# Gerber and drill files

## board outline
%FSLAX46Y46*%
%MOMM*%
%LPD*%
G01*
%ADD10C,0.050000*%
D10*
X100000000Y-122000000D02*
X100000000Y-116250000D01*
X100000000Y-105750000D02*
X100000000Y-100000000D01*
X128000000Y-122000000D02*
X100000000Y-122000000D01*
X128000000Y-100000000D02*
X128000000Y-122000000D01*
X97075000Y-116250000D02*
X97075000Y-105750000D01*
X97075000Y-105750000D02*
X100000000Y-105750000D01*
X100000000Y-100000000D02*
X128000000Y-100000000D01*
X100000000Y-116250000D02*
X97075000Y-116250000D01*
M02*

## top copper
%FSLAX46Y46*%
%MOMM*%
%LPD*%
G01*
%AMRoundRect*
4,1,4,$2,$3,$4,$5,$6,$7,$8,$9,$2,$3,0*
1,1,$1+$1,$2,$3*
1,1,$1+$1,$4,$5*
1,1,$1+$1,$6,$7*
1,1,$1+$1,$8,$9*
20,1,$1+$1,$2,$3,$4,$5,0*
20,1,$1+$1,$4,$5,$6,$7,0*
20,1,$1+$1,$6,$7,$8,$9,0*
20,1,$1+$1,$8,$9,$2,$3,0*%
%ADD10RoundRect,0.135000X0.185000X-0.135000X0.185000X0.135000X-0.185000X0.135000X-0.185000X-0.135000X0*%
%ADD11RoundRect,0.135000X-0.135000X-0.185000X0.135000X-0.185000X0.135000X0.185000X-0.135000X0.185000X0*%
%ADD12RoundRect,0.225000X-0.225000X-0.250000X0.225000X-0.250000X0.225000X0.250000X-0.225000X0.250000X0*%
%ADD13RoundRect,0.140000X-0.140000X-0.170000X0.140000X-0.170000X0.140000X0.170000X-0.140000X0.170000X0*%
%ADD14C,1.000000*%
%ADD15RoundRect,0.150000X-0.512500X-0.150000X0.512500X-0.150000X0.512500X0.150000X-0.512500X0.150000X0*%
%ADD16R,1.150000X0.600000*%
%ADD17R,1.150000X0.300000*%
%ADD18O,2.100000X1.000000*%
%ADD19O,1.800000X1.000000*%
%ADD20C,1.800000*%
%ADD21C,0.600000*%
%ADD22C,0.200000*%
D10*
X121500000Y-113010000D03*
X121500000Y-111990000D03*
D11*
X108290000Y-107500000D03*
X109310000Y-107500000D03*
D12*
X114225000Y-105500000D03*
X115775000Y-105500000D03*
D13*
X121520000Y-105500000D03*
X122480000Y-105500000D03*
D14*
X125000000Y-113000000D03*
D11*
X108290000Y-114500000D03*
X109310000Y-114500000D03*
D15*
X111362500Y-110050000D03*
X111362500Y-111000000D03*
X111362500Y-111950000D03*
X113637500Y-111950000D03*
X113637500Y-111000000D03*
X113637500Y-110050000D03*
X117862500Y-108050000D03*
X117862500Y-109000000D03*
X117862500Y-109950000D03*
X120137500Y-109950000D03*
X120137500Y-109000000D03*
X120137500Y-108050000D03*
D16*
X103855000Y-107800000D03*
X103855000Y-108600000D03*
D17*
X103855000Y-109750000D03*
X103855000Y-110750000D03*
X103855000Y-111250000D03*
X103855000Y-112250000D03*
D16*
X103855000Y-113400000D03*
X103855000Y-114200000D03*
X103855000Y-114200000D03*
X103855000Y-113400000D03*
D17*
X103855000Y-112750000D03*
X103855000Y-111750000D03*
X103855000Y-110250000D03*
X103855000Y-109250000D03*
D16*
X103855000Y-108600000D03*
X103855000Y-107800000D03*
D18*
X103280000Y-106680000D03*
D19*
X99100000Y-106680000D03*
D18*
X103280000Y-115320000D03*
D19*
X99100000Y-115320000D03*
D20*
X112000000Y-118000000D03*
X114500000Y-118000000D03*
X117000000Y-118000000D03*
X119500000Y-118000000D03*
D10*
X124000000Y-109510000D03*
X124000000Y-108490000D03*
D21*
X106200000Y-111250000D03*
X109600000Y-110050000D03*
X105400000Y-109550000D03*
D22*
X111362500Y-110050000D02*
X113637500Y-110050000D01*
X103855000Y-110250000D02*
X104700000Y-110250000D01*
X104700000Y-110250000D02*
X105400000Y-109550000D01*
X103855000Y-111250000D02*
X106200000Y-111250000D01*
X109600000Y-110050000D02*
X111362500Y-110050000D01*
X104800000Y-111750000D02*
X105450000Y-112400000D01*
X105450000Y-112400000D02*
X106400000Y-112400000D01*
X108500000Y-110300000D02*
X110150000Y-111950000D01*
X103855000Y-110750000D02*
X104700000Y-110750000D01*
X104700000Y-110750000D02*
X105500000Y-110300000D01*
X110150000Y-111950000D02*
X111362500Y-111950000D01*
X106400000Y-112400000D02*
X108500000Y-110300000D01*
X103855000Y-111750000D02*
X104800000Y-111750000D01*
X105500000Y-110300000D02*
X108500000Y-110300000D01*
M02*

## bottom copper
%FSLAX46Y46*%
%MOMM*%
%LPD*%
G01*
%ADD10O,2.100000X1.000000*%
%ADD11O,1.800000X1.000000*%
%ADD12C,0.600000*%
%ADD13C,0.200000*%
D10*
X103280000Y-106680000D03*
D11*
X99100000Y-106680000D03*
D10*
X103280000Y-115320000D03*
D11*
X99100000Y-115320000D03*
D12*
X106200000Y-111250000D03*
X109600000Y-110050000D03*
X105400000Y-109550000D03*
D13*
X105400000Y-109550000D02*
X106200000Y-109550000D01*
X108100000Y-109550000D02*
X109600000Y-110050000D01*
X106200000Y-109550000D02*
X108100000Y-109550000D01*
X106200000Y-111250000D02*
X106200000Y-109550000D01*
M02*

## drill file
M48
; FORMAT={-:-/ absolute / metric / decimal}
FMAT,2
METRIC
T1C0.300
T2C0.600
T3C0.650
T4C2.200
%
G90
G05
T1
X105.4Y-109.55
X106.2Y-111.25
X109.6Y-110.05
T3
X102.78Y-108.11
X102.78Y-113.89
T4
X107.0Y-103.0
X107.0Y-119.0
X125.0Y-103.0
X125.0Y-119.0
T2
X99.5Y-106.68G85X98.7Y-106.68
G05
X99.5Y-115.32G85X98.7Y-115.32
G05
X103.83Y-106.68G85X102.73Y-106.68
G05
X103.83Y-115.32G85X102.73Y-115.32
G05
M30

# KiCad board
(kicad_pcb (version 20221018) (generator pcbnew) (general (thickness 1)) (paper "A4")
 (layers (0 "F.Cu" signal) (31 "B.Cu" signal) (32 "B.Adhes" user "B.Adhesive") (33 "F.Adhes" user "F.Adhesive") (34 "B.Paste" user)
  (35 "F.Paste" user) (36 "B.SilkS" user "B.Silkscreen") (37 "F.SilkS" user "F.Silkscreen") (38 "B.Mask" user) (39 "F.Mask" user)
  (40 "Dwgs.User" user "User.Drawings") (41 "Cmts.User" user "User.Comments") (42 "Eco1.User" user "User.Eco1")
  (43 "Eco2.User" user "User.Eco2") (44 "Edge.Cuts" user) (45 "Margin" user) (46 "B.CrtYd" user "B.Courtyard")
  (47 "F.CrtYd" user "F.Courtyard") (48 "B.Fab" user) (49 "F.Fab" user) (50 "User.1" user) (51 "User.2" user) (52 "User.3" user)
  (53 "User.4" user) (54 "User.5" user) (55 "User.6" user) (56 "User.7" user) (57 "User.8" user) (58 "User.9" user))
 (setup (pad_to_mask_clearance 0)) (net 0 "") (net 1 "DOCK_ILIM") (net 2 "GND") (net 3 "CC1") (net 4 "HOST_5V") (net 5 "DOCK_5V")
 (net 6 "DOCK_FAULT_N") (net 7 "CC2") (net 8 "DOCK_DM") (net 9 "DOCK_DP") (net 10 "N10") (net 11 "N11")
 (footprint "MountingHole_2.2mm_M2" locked (layer "F.Cu") (at 107 119)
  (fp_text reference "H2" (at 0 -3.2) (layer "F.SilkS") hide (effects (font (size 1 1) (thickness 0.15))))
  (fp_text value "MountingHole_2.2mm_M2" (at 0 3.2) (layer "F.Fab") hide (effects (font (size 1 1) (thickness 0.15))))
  (pad "" np_thru_hole circle locked (at 0 0) (size 2.2 2.2) (drill 2.2) (layers "*.Cu" "*.Mask")))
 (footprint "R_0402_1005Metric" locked (layer "F.Cu") (at 121.5 112.5 90)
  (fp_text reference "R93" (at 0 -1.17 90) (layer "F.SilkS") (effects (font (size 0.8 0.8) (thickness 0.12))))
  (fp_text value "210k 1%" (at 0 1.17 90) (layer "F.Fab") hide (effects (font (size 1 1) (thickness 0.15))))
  (pad "1" smd roundrect locked (at -0.51 0 90) (size 0.54 0.64) (layers "F.Cu" "F.Paste" "F.Mask") (roundrect_rratio 0.25)
   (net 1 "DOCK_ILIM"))
  (pad "2" smd roundrect locked (at 0.51 0 90) (size 0.54 0.64) (layers "F.Cu" "F.Paste" "F.Mask") (roundrect_rratio 0.25) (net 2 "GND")))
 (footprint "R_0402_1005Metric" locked (layer "F.Cu") (at 108.8 107.5)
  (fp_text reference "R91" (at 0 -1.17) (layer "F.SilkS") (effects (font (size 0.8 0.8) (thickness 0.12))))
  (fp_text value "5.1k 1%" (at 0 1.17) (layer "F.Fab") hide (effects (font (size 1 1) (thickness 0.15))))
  (pad "1" smd roundrect locked (at -0.51 0) (size 0.54 0.64) (layers "F.Cu" "F.Paste" "F.Mask") (roundrect_rratio 0.25) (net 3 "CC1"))
  (pad "2" smd roundrect locked (at 0.51 0) (size 0.54 0.64) (layers "F.Cu" "F.Paste" "F.Mask") (roundrect_rratio 0.25) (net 2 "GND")))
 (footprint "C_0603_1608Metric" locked (layer "F.Cu") (at 115 105.5)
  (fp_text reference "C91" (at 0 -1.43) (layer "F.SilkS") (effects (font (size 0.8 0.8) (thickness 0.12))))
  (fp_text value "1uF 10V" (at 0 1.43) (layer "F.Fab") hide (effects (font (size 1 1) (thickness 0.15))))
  (pad "1" smd roundrect locked (at -0.775 0) (size 0.9 0.95) (layers "F.Cu" "F.Paste" "F.Mask") (roundrect_rratio 0.25) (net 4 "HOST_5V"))
  (pad "2" smd roundrect locked (at 0.775 0) (size 0.9 0.95) (layers "F.Cu" "F.Paste" "F.Mask") (roundrect_rratio 0.25) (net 2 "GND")))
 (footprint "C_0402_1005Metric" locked (layer "F.Cu") (at 122 105.5)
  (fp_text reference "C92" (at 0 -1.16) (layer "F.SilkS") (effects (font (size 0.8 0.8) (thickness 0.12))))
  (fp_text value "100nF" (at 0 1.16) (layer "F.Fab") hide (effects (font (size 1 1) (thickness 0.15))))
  (pad "1" smd roundrect locked (at -0.48 0) (size 0.56 0.62) (layers "F.Cu" "F.Paste" "F.Mask") (roundrect_rratio 0.25) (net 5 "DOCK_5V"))
  (pad "2" smd roundrect locked (at 0.48 0) (size 0.56 0.62) (layers "F.Cu" "F.Paste" "F.Mask") (roundrect_rratio 0.25) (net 2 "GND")))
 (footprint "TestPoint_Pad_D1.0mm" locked (layer "F.Cu") (at 125 113)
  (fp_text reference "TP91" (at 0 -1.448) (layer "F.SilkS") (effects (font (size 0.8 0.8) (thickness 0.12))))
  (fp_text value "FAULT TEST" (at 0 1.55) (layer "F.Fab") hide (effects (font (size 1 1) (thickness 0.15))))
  (pad "1" smd circle locked (at 0 0) (size 1 1) (layers "F.Cu" "F.Mask") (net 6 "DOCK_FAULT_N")))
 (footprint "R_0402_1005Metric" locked (layer "F.Cu") (at 108.8 114.5)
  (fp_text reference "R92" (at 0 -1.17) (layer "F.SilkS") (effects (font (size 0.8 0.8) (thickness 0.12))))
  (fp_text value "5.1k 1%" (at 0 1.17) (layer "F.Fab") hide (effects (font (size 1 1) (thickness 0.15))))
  (pad "1" smd roundrect locked (at -0.51 0) (size 0.54 0.64) (layers "F.Cu" "F.Paste" "F.Mask") (roundrect_rratio 0.25) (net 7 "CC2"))
  (pad "2" smd roundrect locked (at 0.51 0) (size 0.54 0.64) (layers "F.Cu" "F.Paste" "F.Mask") (roundrect_rratio 0.25) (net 2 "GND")))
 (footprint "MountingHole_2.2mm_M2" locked (layer "F.Cu") (at 107 103)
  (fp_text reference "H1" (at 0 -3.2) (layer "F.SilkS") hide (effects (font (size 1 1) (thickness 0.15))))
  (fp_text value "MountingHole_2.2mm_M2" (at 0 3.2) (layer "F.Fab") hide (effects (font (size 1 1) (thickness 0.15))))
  (pad "" np_thru_hole circle locked (at 0 0) (size 2.2 2.2) (drill 2.2) (layers "*.Cu" "*.Mask")))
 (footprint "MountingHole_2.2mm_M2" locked (layer "F.Cu") (at 125 119)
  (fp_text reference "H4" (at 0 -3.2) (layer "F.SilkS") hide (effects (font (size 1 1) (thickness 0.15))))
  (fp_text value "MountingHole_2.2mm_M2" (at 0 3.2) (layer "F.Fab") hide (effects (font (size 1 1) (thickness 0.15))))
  (pad "" np_thru_hole circle locked (at 0 0) (size 2.2 2.2) (drill 2.2) (layers "*.Cu" "*.Mask")))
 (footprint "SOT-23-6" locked (layer "F.Cu") (at 112.5 111)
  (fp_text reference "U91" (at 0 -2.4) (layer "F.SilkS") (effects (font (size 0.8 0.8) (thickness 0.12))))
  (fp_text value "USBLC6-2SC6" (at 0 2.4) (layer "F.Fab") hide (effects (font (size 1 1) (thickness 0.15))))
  (pad "1" smd roundrect locked (at -1.1375 -0.95) (size 1.325 0.6) (layers "F.Cu" "F.Paste" "F.Mask") (roundrect_rratio 0.25)
   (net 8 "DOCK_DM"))
  (pad "2" smd roundrect locked (at -1.1375 0) (size 1.325 0.6) (layers "F.Cu" "F.Paste" "F.Mask") (roundrect_rratio 0.25) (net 2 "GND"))
  (pad "3" smd roundrect locked (at -1.1375 0.95) (size 1.325 0.6) (layers "F.Cu" "F.Paste" "F.Mask") (roundrect_rratio 0.25)
   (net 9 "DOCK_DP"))
  (pad "4" smd roundrect locked (at 1.1375 0.95) (size 1.325 0.6) (layers "F.Cu" "F.Paste" "F.Mask") (roundrect_rratio 0.25)
   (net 9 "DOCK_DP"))
  (pad "5" smd roundrect locked (at 1.1375 0) (size 1.325 0.6) (layers "F.Cu" "F.Paste" "F.Mask") (roundrect_rratio 0.25) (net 4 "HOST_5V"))
  (pad "6" smd roundrect locked (at 1.1375 -0.95) (size 1.325 0.6) (layers "F.Cu" "F.Paste" "F.Mask") (roundrect_rratio 0.25)
   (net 8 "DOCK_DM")))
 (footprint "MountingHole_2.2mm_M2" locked (layer "F.Cu") (at 125 103)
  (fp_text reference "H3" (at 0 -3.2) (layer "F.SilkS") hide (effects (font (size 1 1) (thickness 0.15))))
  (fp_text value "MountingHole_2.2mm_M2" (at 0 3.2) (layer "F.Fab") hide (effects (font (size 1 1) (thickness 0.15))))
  (pad "" np_thru_hole circle locked (at 0 0) (size 2.2 2.2) (drill 2.2) (layers "*.Cu" "*.Mask")))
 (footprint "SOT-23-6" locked (layer "F.Cu") (at 119 109)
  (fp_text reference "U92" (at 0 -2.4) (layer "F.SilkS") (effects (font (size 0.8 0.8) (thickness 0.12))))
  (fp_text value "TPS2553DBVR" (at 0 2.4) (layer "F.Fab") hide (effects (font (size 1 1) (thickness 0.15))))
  (pad "1" smd roundrect locked (at -1.1375 -0.95) (size 1.325 0.6) (layers "F.Cu" "F.Paste" "F.Mask") (roundrect_rratio 0.25)
   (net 4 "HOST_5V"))
  (pad "2" smd roundrect locked (at -1.1375 0) (size 1.325 0.6) (layers "F.Cu" "F.Paste" "F.Mask") (roundrect_rratio 0.25) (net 2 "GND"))
  (pad "3" smd roundrect locked (at -1.1375 0.95) (size 1.325 0.6) (layers "F.Cu" "F.Paste" "F.Mask") (roundrect_rratio 0.25)
   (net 4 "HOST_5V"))
  (pad "4" smd roundrect locked (at 1.1375 0.95) (size 1.325 0.6) (layers "F.Cu" "F.Paste" "F.Mask") (roundrect_rratio 0.25)
   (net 6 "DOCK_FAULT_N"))
  (pad "5" smd roundrect locked (at 1.1375 0) (size 1.325 0.6) (layers "F.Cu" "F.Paste" "F.Mask") (roundrect_rratio 0.25)
   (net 1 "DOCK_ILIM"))
  (pad "6" smd roundrect locked (at 1.1375 -0.95) (size 1.325 0.6) (layers "F.Cu" "F.Paste" "F.Mask") (roundrect_rratio 0.25)
   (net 5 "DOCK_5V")))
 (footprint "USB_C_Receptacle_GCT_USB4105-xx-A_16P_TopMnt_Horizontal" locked (layer "F.Cu") (at 100.175 111 -90)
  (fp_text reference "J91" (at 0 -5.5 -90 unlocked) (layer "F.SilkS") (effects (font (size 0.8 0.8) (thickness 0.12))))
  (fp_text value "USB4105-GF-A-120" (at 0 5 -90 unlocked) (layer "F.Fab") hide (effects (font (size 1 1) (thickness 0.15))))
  (pad "" np_thru_hole circle locked (at -2.89 -2.605 270) (size 0.65 0.65) (drill 0.65) (layers "F&B.Cu" "*.Mask"))
  (pad "" np_thru_hole circle locked (at 2.89 -2.605 270) (size 0.65 0.65) (drill 0.65) (layers "F&B.Cu" "*.Mask"))
  (pad "A1" smd rect locked (at -3.2 -3.68 270) (size 0.6 1.15) (layers "F.Cu" "F.Paste" "F.Mask") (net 2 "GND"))
  (pad "A4" smd rect locked (at -2.4 -3.68 270) (size 0.6 1.15) (layers "F.Cu" "F.Paste" "F.Mask") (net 4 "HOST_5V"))
  (pad "A5" smd rect locked (at -1.25 -3.68 270) (size 0.3 1.15) (layers "F.Cu" "F.Paste" "F.Mask") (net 3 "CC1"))
  (pad "A6" smd rect locked (at -0.25 -3.68 270) (size 0.3 1.15) (layers "F.Cu" "F.Paste" "F.Mask") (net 9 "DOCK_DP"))
  (pad "A7" smd rect locked (at 0.25 -3.68 270) (size 0.3 1.15) (layers "F.Cu" "F.Paste" "F.Mask") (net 8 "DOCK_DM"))
  (pad "A8" smd rect locked (at 1.25 -3.68 270) (size 0.3 1.15) (layers "F.Cu" "F.Paste" "F.Mask") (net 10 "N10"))
  (pad "A9" smd rect locked (at 2.4 -3.68 270) (size 0.6 1.15) (layers "F.Cu" "F.Paste" "F.Mask") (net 4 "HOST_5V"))
  (pad "A12" smd rect locked (at 3.2 -3.68 270) (size 0.6 1.15) (layers "F.Cu" "F.Paste" "F.Mask") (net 2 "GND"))
  (pad "B1" smd rect locked (at 3.2 -3.68 270) (size 0.6 1.15) (layers "F.Cu" "F.Paste" "F.Mask") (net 2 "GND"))
  (pad "B4" smd rect locked (at 2.4 -3.68 270) (size 0.6 1.15) (layers "F.Cu" "F.Paste" "F.Mask") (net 4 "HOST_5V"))
  (pad "B5" smd rect locked (at 1.75 -3.68 270) (size 0.3 1.15) (layers "F.Cu" "F.Paste" "F.Mask") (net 7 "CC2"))
  (pad "B6" smd rect locked (at 0.75 -3.68 270) (size 0.3 1.15) (layers "F.Cu" "F.Paste" "F.Mask") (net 9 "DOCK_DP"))
  (pad "B7" smd rect locked (at -0.75 -3.68 270) (size 0.3 1.15) (layers "F.Cu" "F.Paste" "F.Mask") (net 8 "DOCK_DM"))
  (pad "B8" smd rect locked (at -1.75 -3.68 270) (size 0.3 1.15) (layers "F.Cu" "F.Paste" "F.Mask") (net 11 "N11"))
  (pad "B9" smd rect locked (at -2.4 -3.68 270) (size 0.6 1.15) (layers "F.Cu" "F.Paste" "F.Mask") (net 4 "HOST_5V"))
  (pad "B12" smd rect locked (at -3.2 -3.68 270) (size 0.6 1.15) (layers "F.Cu" "F.Paste" "F.Mask") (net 2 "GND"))
  (pad "S1" thru_hole oval locked (at -4.32 -3.105 270) (size 1 2.1) (drill oval 0.6 1.7) (layers "*.Cu" "*.Mask" "F.Paste") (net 2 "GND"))
  (pad "S1" thru_hole oval locked (at -4.32 1.075 270) (size 1 1.8) (drill oval 0.6 1.4) (layers "*.Cu" "*.Mask" "F.Paste") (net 2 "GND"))
  (pad "S1" thru_hole oval locked (at 4.32 -3.105 270) (size 1 2.1) (drill oval 0.6 1.7) (layers "*.Cu" "*.Mask" "F.Paste") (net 2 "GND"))
  (pad "S1" thru_hole oval locked (at 4.32 1.075 270) (size 1 1.8) (drill oval 0.6 1.4) (layers "*.Cu" "*.Mask" "F.Paste") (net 2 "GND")))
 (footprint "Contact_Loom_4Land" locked (layer "F.Cu") (at 112 118)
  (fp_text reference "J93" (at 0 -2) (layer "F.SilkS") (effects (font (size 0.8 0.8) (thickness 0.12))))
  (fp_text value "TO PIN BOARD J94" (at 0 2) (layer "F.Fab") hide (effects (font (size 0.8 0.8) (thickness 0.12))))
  (pad "1" smd circle locked (at 0 0) (size 1.8 1.8) (layers "F.Cu" "F.Paste" "F.Mask") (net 2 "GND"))
  (pad "2" smd circle locked (at 2.5 0) (size 1.8 1.8) (layers "F.Cu" "F.Paste" "F.Mask") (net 8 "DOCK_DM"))
  (pad "3" smd circle locked (at 5 0) (size 1.8 1.8) (layers "F.Cu" "F.Paste" "F.Mask") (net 9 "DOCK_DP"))
  (pad "4" smd circle locked (at 7.5 0) (size 1.8 1.8) (layers "F.Cu" "F.Paste" "F.Mask") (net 5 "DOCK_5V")))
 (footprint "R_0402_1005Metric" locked (layer "F.Cu") (at 124 109 90)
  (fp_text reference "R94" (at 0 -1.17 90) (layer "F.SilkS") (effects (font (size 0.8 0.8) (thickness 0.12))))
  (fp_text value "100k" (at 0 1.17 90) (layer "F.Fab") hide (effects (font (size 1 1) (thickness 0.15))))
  (pad "1" smd roundrect locked (at -0.51 0 90) (size 0.54 0.64) (layers "F.Cu" "F.Paste" "F.Mask") (roundrect_rratio 0.25)
   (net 4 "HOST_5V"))
  (pad "2" smd roundrect locked (at 0.51 0 90) (size 0.54 0.64) (layers "F.Cu" "F.Paste" "F.Mask") (roundrect_rratio 0.25)
   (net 6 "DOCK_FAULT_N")))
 (gr_line (start 100 122) (end 100 116.25) (stroke (width 0.05) (type default)) (layer "Edge.Cuts"))
 (gr_line (start 100 105.75) (end 100 100) (stroke (width 0.05) (type default)) (layer "Edge.Cuts"))
 (gr_line (start 128 122) (end 100 122) (stroke (width 0.05) (type default)) (layer "Edge.Cuts"))
 (gr_line (start 128 100) (end 128 122) (stroke (width 0.05) (type default)) (layer "Edge.Cuts"))
 (gr_line (start 97.075 116.25) (end 97.075 105.75) (stroke (width 0.05) (type default)) (layer "Edge.Cuts"))
 (gr_line (start 97.075 105.75) (end 100 105.75) (stroke (width 0.05) (type default)) (layer "Edge.Cuts"))
 (gr_line (start 100 100) (end 128 100) (stroke (width 0.05) (type default)) (layer "Edge.Cuts"))
 (gr_line (start 100 116.25) (end 97.075 116.25) (stroke (width 0.05) (type default)) (layer "Edge.Cuts"))
 (segment locked (start 111.3625 110.05) (end 113.6375 110.05) (width 0.2) (layer "F.Cu") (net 8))
 (segment locked (start 103.855 110.25) (end 104.7 110.25) (width 0.2) (layer "F.Cu") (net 8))
 (segment locked (start 104.7 110.25) (end 105.4 109.55) (width 0.2) (layer "F.Cu") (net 8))
 (segment locked (start 103.855 111.25) (end 106.2 111.25) (width 0.2) (layer "F.Cu") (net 8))
 (segment locked (start 109.6 110.05) (end 111.3625 110.05) (width 0.2) (layer "F.Cu") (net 8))
 (via locked (at 106.2 111.25) (size 0.6) (drill 0.3) (layers "F.Cu" "B.Cu") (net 8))
 (via locked (at 109.6 110.05) (size 0.6) (drill 0.3) (layers "F.Cu" "B.Cu") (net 8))
 (via locked (at 105.4 109.55) (size 0.6) (drill 0.3) (layers "F.Cu" "B.Cu") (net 8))
 (segment locked (start 105.4 109.55) (end 106.2 109.55) (width 0.2) (layer "B.Cu") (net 8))
 (segment locked (start 108.1 109.55) (end 109.6 110.05) (width 0.2) (layer "B.Cu") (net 8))
 (segment locked (start 106.2 109.55) (end 108.1 109.55) (width 0.2) (layer "B.Cu") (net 8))
 (segment locked (start 106.2 111.25) (end 106.2 109.55) (width 0.2) (layer "B.Cu") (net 8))
 (segment locked (start 104.8 111.75) (end 105.45 112.4) (width 0.2) (layer "F.Cu") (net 9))
 (segment locked (start 105.45 112.4) (end 106.4 112.4) (width 0.2) (layer "F.Cu") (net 9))
 (segment locked (start 108.5 110.3) (end 110.15 111.95) (width 0.2) (layer "F.Cu") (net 9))
 (segment locked (start 103.855 110.75) (end 104.7 110.75) (width 0.2) (layer "F.Cu") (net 9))
 (segment locked (start 104.7 110.75) (end 105.5 110.3) (width 0.2) (layer "F.Cu") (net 9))
 (segment locked (start 110.15 111.95) (end 111.3625 111.95) (width 0.2) (layer "F.Cu") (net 9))
 (segment locked (start 106.4 112.4) (end 108.5 110.3) (width 0.2) (layer "F.Cu") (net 9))
 (segment locked (start 103.855 111.75) (end 104.8 111.75) (width 0.2) (layer "F.Cu") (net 9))
 (segment locked (start 105.5 110.3) (end 108.5 110.3) (width 0.2) (layer "F.Cu") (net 9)))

